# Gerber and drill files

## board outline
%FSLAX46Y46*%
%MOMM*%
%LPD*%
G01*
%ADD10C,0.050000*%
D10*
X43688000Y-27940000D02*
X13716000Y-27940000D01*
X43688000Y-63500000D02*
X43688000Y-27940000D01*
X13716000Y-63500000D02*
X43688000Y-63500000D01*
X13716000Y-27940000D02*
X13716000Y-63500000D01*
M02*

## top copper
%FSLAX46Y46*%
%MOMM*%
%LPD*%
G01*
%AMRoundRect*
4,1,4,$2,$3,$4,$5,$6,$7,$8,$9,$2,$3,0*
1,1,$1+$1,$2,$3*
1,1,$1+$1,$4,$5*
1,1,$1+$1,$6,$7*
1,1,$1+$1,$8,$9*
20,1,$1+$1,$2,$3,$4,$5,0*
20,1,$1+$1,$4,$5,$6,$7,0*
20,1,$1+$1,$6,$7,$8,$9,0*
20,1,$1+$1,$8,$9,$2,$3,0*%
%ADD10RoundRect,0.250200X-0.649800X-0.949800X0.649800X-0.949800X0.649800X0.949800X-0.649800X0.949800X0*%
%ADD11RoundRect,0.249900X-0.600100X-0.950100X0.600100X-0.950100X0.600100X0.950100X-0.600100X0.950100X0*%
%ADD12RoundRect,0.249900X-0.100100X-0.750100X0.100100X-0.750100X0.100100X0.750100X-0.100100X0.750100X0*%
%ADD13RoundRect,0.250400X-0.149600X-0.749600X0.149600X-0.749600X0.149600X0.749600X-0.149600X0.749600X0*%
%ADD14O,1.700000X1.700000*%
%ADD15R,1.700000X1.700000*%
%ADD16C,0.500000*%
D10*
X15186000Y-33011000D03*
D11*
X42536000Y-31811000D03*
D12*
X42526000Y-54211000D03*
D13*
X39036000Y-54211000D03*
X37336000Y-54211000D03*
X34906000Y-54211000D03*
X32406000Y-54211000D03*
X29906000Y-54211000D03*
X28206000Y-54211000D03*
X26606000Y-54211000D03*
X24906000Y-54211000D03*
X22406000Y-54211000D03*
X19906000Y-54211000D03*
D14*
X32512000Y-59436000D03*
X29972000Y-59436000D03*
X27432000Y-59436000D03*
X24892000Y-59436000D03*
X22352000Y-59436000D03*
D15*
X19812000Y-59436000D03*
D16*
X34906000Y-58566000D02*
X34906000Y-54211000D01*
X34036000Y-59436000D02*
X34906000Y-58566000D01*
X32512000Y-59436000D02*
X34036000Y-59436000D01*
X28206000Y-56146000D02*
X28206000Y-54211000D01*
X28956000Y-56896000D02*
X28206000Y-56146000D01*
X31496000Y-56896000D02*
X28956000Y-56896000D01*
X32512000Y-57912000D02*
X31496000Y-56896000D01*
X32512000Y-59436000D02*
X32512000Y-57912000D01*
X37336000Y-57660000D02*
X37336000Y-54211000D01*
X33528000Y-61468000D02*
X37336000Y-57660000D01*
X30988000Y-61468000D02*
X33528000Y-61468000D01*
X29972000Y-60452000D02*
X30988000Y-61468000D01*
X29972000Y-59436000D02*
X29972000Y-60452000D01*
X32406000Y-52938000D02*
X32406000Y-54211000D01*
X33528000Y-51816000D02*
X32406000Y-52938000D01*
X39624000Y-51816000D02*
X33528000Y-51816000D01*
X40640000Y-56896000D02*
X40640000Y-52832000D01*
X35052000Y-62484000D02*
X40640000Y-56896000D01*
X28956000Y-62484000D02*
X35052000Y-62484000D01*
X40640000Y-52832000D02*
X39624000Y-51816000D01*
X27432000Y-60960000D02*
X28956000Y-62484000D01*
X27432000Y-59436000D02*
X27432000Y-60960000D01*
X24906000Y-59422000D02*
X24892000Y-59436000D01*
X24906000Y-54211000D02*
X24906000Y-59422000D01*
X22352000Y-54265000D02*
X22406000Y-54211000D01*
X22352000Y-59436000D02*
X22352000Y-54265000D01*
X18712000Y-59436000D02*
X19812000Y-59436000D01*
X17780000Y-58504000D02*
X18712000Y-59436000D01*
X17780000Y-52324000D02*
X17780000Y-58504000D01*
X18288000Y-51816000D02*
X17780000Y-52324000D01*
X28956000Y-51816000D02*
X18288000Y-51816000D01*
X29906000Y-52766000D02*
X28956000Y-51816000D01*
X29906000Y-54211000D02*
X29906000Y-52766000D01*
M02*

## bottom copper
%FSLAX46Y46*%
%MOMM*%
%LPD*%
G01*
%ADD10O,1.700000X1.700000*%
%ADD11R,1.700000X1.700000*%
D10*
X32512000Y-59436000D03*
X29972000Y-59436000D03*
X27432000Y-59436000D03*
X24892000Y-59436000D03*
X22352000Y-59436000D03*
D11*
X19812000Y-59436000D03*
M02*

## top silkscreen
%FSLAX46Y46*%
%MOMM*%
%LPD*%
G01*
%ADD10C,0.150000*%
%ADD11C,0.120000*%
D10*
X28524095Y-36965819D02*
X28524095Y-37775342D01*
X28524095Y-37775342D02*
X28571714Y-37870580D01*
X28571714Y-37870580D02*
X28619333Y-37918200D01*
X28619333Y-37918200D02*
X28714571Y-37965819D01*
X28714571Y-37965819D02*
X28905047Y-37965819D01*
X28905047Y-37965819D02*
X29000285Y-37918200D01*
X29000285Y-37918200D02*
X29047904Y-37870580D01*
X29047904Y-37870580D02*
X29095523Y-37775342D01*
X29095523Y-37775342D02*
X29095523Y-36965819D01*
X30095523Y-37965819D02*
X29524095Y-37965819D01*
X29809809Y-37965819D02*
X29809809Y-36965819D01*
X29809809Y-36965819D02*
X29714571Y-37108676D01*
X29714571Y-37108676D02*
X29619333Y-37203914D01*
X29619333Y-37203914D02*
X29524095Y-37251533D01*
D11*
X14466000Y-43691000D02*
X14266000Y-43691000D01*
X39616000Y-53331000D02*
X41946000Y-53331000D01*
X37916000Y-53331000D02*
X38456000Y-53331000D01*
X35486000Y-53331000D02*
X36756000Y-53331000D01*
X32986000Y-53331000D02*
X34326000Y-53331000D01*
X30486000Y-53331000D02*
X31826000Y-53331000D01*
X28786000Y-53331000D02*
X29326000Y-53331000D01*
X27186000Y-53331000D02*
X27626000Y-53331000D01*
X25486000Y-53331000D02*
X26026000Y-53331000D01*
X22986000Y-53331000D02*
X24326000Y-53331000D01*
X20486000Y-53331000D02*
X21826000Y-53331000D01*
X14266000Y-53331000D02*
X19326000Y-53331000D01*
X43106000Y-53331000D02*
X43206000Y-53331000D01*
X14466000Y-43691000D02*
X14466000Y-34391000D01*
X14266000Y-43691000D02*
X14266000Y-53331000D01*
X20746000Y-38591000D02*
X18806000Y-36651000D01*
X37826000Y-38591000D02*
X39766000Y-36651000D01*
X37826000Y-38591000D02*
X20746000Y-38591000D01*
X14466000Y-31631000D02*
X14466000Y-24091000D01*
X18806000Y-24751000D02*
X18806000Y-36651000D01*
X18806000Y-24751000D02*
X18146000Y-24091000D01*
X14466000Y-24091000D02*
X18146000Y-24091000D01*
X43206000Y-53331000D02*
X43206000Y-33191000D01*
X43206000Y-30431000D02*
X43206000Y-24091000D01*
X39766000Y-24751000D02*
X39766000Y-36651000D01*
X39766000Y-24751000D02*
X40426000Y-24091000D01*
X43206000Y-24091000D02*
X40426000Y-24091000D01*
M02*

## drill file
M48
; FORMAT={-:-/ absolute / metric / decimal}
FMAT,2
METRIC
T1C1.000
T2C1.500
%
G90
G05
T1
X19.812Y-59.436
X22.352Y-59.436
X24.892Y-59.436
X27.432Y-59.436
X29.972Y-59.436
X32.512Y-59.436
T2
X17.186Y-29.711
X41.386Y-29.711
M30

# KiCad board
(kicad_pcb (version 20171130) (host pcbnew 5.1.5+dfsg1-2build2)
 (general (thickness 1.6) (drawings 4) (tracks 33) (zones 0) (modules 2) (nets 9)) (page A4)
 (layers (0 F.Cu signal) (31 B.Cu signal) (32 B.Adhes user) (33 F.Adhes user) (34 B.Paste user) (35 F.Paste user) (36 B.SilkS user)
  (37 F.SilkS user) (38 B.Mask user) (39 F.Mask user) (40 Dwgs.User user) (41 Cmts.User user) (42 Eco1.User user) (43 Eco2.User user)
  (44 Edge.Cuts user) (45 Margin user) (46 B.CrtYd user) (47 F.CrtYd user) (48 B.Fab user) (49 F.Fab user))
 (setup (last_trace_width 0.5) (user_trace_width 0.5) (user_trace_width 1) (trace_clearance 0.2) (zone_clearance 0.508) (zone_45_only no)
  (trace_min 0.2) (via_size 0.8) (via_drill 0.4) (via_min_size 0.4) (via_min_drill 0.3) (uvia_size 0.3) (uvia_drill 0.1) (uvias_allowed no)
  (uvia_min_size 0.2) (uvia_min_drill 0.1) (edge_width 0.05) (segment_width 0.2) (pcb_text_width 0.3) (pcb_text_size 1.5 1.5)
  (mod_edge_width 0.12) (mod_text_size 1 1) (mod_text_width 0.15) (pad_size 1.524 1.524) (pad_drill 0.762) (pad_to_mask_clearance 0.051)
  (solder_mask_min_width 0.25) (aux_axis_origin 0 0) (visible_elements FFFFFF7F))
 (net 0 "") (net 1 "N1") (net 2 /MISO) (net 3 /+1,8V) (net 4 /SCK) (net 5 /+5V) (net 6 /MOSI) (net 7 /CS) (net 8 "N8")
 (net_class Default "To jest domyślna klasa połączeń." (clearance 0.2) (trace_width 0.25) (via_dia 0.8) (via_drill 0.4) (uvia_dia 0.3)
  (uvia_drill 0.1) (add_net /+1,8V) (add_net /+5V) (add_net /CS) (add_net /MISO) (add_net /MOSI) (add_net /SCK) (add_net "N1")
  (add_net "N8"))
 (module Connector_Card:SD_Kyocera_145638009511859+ (layer F.Cu) (at 29.286 47.011)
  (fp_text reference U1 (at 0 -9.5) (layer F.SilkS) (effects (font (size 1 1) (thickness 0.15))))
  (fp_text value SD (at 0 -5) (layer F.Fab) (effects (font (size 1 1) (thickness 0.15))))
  (fp_line (start -14.82 -3.32) (end -15.02 -3.32) (layer F.SilkS) (width 0.12))
  (fp_line (start 10.33 6.32) (end 12.66 6.32) (layer F.SilkS) (width 0.12))
  (fp_line (start 8.63 6.32) (end 9.17 6.32) (layer F.SilkS) (width 0.12))
  (fp_line (start 6.2 6.32) (end 7.47 6.32) (layer F.SilkS) (width 0.12))
  (fp_line (start 3.7 6.32) (end 5.04 6.32) (layer F.SilkS) (width 0.12))
  (fp_line (start 1.2 6.32) (end 2.54 6.32) (layer F.SilkS) (width 0.12))
  (fp_line (start -0.5 6.32) (end 0.04 6.32) (layer F.SilkS) (width 0.12))
  (fp_line (start -2.1 6.32) (end -1.66 6.32) (layer F.SilkS) (width 0.12))
  (fp_line (start -3.8 6.32) (end -3.26 6.32) (layer F.SilkS) (width 0.12))
  (fp_line (start -6.3 6.32) (end -4.96 6.32) (layer F.SilkS) (width 0.12))
  (fp_line (start -8.8 6.32) (end -7.46 6.32) (layer F.SilkS) (width 0.12))
  (fp_line (start -15.02 6.32) (end -9.96 6.32) (layer F.SilkS) (width 0.12))
  (fp_line (start 13.82 6.32) (end 13.92 6.32) (layer F.SilkS) (width 0.12))
  (fp_line (start -14.82 -3.32) (end -14.82 -12.62) (layer F.SilkS) (width 0.12))
  (fp_line (start -15.02 -3.32) (end -15.02 6.32) (layer F.SilkS) (width 0.12))
  (fp_line (start -8.54 -8.42) (end -10.48 -10.36) (layer F.SilkS) (width 0.12))
  (fp_line (start 8.54 -8.42) (end 10.48 -10.36) (layer F.SilkS) (width 0.12))
  (fp_line (start 8.54 -8.42) (end -8.54 -8.42) (layer F.SilkS) (width 0.12))
  (fp_line (start -14.82 -15.38) (end -14.82 -22.92) (layer F.SilkS) (width 0.12))
  (fp_line (start -10.48 -22.26) (end -10.48 -10.36) (layer F.SilkS) (width 0.12))
  (fp_line (start -10.48 -22.26) (end -11.14 -22.92) (layer F.SilkS) (width 0.12))
  (fp_line (start -14.82 -22.92) (end -11.14 -22.92) (layer F.SilkS) (width 0.12))
  (fp_line (start 13.92 6.32) (end 13.92 -13.82) (layer F.SilkS) (width 0.12))
  (fp_line (start 13.92 -16.58) (end 13.92 -22.92) (layer F.SilkS) (width 0.12))
  (fp_line (start 10.48 -22.26) (end 10.48 -10.36) (layer F.SilkS) (width 0.12))
  (fp_line (start 10.48 -22.26) (end 11.14 -22.92) (layer F.SilkS) (width 0.12))
  (fp_line (start 13.92 -22.92) (end 11.14 -22.92) (layer F.SilkS) (width 0.12))
  (pad "" smd roundrect (at -14.1 -14) (size 1.8 2.4) (layers F.Cu F.Paste F.Mask) (roundrect_rratio 0.139))
  (pad SH smd roundrect (at 13.25 -15.2) (size 1.7 2.4) (layers F.Cu F.Paste F.Mask) (roundrect_rratio 0.147))
  (pad "" np_thru_hole circle (at -12.1 -17.3) (size 1.5 1.5) (drill 1.5) (layers *.Cu *.Mask))
  (pad "" np_thru_hole circle (at 12.1 -17.3) (size 1.5 1.5) (drill 1.5) (layers *.Cu *.Mask))
  (pad 11 smd roundrect (at 13.24 7.2) (size 0.7 2) (layers F.Cu F.Paste F.Mask) (roundrect_rratio 0.357))
  (pad 8 smd roundrect (at 9.75 7.2) (size 0.8 2) (layers F.Cu F.Paste F.Mask) (roundrect_rratio 0.313) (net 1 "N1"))
  (pad 7 smd roundrect (at 8.05 7.2) (size 0.8 2) (layers F.Cu F.Paste F.Mask) (roundrect_rratio 0.313) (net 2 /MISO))
  (pad 6 smd roundrect (at 5.62 7.2) (size 0.8 2) (layers F.Cu F.Paste F.Mask) (roundrect_rratio 0.313) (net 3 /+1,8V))
  (pad 5 smd roundrect (at 3.12 7.2) (size 0.8 2) (layers F.Cu F.Paste F.Mask) (roundrect_rratio 0.313) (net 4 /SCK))
  (pad 4 smd roundrect (at 0.62 7.2) (size 0.8 2) (layers F.Cu F.Paste F.Mask) (roundrect_rratio 0.313) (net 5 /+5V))
  (pad 3 smd roundrect (at -1.08 7.2) (size 0.8 2) (layers F.Cu F.Paste F.Mask) (roundrect_rratio 0.313) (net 3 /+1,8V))
  (pad 10 smd roundrect (at -2.68 7.2) (size 0.8 2) (layers F.Cu F.Paste F.Mask) (roundrect_rratio 0.313))
  (pad 2 smd roundrect (at -4.38 7.2) (size 0.8 2) (layers F.Cu F.Paste F.Mask) (roundrect_rratio 0.313) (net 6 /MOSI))
  (pad 1 smd roundrect (at -6.88 7.2) (size 0.8 2) (layers F.Cu F.Paste F.Mask) (roundrect_rratio 0.313) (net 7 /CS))
  (pad 9 smd roundrect (at -9.38 7.2) (size 0.8 2) (layers F.Cu F.Paste F.Mask) (roundrect_rratio 0.313) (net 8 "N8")))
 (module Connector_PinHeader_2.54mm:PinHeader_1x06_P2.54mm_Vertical (layer B.Cu) (at 19.812 59.436 270)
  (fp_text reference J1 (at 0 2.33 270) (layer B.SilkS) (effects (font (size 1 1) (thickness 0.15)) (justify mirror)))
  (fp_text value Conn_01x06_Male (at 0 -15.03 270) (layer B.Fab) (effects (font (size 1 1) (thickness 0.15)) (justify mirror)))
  (pad 6 thru_hole oval (at 0 -12.7 270) (size 1.7 1.7) (drill 1) (layers *.Cu *.Mask) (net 3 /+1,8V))
  (pad 5 thru_hole oval (at 0 -10.16 270) (size 1.7 1.7) (drill 1) (layers *.Cu *.Mask) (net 2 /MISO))
  (pad 4 thru_hole oval (at 0 -7.62 270) (size 1.7 1.7) (drill 1) (layers *.Cu *.Mask) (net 4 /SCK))
  (pad 3 thru_hole oval (at 0 -5.08 270) (size 1.7 1.7) (drill 1) (layers *.Cu *.Mask) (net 6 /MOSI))
  (pad 2 thru_hole oval (at 0 -2.54 270) (size 1.7 1.7) (drill 1) (layers *.Cu *.Mask) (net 7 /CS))
  (pad 1 thru_hole rect (at 0 0 270) (size 1.7 1.7) (drill 1) (layers *.Cu *.Mask) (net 5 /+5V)))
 (gr_line (start 43.688 27.94) (end 13.716 27.94) (layer Edge.Cuts) (width 0.05))
 (gr_line (start 43.688 63.5) (end 43.688 27.94) (layer Edge.Cuts) (width 0.05))
 (gr_line (start 13.716 63.5) (end 43.688 63.5) (layer Edge.Cuts) (width 0.05))
 (gr_line (start 13.716 27.94) (end 13.716 63.5) (layer Edge.Cuts) (width 0.05))
 (segment (start 34.906 58.566) (end 34.906 54.211) (width 0.5) (layer F.Cu) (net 3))
 (segment (start 34.036 59.436) (end 34.906 58.566) (width 0.5) (layer F.Cu) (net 3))
 (segment (start 32.512 59.436) (end 34.036 59.436) (width 0.5) (layer F.Cu) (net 3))
 (segment (start 28.206 56.146) (end 28.206 54.211) (width 0.5) (layer F.Cu) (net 3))
 (segment (start 28.956 56.896) (end 28.206 56.146) (width 0.5) (layer F.Cu) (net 3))
 (segment (start 31.496 56.896) (end 28.956 56.896) (width 0.5) (layer F.Cu) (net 3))
 (segment (start 32.512 57.912) (end 31.496 56.896) (width 0.5) (layer F.Cu) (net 3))
 (segment (start 32.512 59.436) (end 32.512 57.912) (width 0.5) (layer F.Cu) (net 3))
 (segment (start 37.336 57.66) (end 37.336 54.211) (width 0.5) (layer F.Cu) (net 2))
 (segment (start 33.528 61.468) (end 37.336 57.66) (width 0.5) (layer F.Cu) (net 2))
 (segment (start 30.988 61.468) (end 33.528 61.468) (width 0.5) (layer F.Cu) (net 2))
 (segment (start 29.972 60.452) (end 30.988 61.468) (width 0.5) (layer F.Cu) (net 2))
 (segment (start 29.972 59.436) (end 29.972 60.452) (width 0.5) (layer F.Cu) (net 2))
 (segment (start 32.406 52.938) (end 32.406 54.211) (width 0.5) (layer F.Cu) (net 4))
 (segment (start 33.528 51.816) (end 32.406 52.938) (width 0.5) (layer F.Cu) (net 4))
 (segment (start 39.624 51.816) (end 33.528 51.816) (width 0.5) (layer F.Cu) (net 4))
 (segment (start 40.64 56.896) (end 40.64 52.832) (width 0.5) (layer F.Cu) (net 4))
 (segment (start 35.052 62.484) (end 40.64 56.896) (width 0.5) (layer F.Cu) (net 4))
 (segment (start 28.956 62.484) (end 35.052 62.484) (width 0.5) (layer F.Cu) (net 4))
 (segment (start 40.64 52.832) (end 39.624 51.816) (width 0.5) (layer F.Cu) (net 4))
 (segment (start 27.432 60.96) (end 28.956 62.484) (width 0.5) (layer F.Cu) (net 4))
 (segment (start 27.432 59.436) (end 27.432 60.96) (width 0.5) (layer F.Cu) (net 4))
 (segment (start 24.906 59.422) (end 24.892 59.436) (width 0.5) (layer F.Cu) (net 6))
 (segment (start 24.906 54.211) (end 24.906 59.422) (width 0.5) (layer F.Cu) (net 6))
 (segment (start 22.352 54.265) (end 22.406 54.211) (width 0.5) (layer F.Cu) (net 7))
 (segment (start 22.352 59.436) (end 22.352 54.265) (width 0.5) (layer F.Cu) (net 7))
 (segment (start 18.712 59.436) (end 19.812 59.436) (width 0.5) (layer F.Cu) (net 5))
 (segment (start 17.78 58.504) (end 18.712 59.436) (width 0.5) (layer F.Cu) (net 5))
 (segment (start 17.78 52.324) (end 17.78 58.504) (width 0.5) (layer F.Cu) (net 5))
 (segment (start 18.288 51.816) (end 17.78 52.324) (width 0.5) (layer F.Cu) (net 5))
 (segment (start 28.956 51.816) (end 18.288 51.816) (width 0.5) (layer F.Cu) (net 5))
 (segment (start 29.906 52.766) (end 28.956 51.816) (width 0.5) (layer F.Cu) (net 5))
 (segment (start 29.906 54.211) (end 29.906 52.766) (width 0.5) (layer F.Cu) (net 5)))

